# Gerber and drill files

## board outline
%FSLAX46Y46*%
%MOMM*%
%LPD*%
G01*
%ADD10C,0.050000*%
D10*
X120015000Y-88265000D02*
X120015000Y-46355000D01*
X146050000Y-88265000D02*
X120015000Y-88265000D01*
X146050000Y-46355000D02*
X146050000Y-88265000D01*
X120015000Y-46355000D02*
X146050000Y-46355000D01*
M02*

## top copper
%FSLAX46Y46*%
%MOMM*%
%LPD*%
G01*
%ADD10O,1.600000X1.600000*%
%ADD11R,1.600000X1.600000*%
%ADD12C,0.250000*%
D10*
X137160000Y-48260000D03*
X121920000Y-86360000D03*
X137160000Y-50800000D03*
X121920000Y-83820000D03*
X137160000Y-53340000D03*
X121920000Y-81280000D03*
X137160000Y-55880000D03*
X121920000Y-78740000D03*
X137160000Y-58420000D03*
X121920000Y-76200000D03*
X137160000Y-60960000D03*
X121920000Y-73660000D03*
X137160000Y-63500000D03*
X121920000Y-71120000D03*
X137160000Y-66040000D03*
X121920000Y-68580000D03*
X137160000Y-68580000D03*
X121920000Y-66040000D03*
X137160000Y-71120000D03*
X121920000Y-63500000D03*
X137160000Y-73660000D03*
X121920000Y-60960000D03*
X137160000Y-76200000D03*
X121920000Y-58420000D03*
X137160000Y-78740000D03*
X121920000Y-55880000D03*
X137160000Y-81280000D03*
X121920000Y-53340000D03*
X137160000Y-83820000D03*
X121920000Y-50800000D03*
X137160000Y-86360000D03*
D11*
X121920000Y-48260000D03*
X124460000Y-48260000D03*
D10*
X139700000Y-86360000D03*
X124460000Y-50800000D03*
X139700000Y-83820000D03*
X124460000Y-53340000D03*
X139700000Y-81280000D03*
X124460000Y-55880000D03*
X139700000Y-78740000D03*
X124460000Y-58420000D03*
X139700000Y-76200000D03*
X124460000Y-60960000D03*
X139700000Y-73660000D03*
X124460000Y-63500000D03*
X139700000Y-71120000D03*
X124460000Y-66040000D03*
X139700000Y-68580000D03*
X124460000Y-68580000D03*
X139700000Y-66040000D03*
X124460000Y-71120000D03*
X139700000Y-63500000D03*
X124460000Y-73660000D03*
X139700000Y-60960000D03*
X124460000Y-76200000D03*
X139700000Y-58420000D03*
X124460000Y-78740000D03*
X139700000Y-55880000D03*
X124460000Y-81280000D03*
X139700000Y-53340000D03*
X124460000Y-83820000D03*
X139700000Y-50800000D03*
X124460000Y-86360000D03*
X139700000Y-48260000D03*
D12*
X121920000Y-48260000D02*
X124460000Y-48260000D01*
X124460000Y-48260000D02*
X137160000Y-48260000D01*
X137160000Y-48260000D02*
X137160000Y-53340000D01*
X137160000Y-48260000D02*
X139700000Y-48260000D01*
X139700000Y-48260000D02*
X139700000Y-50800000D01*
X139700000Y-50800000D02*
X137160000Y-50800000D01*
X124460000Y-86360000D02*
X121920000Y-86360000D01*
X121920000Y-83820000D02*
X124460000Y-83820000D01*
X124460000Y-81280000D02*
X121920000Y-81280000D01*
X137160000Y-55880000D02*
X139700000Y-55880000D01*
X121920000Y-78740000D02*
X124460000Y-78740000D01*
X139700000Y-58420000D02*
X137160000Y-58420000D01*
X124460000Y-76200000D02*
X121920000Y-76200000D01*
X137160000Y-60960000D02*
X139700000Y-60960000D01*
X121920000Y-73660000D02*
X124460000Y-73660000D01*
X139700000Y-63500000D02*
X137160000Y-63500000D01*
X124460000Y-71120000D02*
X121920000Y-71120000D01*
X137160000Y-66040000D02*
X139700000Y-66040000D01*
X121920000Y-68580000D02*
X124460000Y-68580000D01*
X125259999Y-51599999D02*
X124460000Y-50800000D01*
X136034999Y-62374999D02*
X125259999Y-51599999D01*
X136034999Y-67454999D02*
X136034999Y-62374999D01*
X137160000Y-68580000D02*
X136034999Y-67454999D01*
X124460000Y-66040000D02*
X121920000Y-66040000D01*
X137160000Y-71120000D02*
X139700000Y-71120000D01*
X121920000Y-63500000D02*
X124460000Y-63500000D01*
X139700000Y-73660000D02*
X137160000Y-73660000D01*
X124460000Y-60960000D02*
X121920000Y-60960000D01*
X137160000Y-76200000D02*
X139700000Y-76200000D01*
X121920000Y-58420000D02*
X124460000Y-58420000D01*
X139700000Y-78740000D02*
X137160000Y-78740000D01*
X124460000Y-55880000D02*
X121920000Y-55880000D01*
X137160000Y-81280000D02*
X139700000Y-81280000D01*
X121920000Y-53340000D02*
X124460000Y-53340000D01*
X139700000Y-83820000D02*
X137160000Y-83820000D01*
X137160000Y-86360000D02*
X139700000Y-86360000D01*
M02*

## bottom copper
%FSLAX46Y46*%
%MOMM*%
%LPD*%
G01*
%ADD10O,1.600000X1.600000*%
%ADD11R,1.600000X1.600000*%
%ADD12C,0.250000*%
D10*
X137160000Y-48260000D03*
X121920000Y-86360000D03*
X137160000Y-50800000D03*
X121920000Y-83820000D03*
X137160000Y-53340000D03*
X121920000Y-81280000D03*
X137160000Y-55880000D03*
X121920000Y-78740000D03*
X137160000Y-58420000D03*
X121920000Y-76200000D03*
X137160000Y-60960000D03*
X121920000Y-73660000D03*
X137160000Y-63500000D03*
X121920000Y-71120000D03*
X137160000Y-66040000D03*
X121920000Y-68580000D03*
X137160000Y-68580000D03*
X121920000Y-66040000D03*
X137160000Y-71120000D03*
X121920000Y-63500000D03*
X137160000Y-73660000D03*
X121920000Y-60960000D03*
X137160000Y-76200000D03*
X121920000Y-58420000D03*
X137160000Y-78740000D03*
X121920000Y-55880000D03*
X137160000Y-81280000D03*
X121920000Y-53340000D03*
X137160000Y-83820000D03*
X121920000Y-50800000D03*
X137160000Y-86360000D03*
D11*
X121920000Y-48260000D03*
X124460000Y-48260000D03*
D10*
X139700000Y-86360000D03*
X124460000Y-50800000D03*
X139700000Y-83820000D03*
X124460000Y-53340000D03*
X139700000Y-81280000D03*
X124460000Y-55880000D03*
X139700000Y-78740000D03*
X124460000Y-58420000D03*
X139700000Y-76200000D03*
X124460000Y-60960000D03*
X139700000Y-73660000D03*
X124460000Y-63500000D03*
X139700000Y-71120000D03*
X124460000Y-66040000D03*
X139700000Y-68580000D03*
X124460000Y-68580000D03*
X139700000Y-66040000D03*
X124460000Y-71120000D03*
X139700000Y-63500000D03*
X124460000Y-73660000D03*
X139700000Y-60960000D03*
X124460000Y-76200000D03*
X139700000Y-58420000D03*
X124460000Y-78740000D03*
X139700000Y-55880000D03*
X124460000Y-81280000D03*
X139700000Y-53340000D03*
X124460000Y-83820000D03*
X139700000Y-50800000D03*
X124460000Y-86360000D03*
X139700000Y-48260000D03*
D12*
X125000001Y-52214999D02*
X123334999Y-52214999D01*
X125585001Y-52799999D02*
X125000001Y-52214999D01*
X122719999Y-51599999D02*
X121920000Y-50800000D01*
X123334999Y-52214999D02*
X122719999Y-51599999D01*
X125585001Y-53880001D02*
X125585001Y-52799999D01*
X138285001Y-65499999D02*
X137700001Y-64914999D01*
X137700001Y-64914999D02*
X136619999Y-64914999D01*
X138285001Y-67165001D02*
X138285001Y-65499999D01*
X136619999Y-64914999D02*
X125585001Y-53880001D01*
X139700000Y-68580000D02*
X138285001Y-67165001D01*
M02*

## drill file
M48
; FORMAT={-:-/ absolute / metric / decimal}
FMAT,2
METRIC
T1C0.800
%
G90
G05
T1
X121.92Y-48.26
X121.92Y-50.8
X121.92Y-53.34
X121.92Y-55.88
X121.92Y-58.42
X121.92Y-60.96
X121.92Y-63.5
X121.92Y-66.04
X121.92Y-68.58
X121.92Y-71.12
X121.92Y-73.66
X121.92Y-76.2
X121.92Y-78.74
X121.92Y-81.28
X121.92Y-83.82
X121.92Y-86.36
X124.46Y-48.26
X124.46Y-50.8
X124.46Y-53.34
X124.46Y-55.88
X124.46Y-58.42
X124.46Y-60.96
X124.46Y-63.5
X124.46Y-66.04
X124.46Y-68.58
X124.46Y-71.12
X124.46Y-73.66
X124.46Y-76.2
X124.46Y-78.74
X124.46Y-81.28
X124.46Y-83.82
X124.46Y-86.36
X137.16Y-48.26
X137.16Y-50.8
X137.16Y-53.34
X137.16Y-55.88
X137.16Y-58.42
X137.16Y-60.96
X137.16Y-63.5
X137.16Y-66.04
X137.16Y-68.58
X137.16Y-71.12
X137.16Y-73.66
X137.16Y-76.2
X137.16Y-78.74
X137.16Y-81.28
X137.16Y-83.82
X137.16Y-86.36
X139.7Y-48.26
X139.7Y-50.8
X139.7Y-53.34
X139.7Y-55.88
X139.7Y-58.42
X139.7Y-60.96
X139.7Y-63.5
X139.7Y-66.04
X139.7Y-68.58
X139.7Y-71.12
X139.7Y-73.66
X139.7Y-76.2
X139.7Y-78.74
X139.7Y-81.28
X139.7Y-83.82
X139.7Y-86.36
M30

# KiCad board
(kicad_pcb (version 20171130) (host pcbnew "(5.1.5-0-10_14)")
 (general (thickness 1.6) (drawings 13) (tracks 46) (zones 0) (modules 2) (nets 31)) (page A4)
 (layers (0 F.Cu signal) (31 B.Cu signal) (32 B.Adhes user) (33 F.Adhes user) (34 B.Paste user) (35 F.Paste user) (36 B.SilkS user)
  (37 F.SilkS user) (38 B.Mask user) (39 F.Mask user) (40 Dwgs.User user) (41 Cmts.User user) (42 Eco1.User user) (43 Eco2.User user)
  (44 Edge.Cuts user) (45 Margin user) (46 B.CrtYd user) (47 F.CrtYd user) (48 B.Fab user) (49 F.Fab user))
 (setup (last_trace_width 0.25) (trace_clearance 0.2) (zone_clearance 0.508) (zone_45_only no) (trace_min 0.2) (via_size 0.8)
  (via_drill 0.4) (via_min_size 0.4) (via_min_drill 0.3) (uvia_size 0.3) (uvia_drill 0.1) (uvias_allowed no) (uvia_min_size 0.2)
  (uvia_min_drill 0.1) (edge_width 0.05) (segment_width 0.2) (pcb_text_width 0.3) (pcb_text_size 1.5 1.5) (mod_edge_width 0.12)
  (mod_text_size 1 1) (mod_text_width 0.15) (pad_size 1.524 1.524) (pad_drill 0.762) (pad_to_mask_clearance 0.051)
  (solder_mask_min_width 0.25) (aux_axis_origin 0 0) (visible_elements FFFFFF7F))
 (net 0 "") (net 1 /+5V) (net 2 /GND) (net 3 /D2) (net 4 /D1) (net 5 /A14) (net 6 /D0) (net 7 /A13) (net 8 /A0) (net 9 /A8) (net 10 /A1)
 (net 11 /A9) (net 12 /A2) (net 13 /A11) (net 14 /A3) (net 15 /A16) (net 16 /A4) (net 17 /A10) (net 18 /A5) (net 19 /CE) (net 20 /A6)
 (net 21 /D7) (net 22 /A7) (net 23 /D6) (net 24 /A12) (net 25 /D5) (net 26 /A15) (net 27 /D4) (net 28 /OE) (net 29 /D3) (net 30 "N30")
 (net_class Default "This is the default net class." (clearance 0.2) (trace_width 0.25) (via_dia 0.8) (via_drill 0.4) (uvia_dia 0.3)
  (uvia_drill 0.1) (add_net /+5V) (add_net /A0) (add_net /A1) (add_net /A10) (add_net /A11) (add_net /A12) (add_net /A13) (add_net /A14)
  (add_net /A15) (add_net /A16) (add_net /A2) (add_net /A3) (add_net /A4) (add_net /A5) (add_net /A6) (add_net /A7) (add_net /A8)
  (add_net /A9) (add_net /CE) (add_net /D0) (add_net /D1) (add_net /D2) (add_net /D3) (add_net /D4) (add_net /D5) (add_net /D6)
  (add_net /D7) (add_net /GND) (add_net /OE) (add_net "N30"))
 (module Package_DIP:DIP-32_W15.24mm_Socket (layer F.Cu) (at 121.92 48.26)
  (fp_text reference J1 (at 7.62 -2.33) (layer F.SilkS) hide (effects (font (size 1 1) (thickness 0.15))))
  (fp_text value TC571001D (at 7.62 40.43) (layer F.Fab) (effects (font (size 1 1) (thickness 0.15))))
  (pad 32 thru_hole oval (at 15.24 0) (size 1.6 1.6) (drill 0.8) (layers *.Cu *.Mask) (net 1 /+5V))
  (pad 16 thru_hole oval (at 0 38.1) (size 1.6 1.6) (drill 0.8) (layers *.Cu *.Mask) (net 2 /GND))
  (pad 31 thru_hole oval (at 15.24 2.54) (size 1.6 1.6) (drill 0.8) (layers *.Cu *.Mask) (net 1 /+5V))
  (pad 15 thru_hole oval (at 0 35.56) (size 1.6 1.6) (drill 0.8) (layers *.Cu *.Mask) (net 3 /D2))
  (pad 30 thru_hole oval (at 15.24 5.08) (size 1.6 1.6) (drill 0.8) (layers *.Cu *.Mask) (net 1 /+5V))
  (pad 14 thru_hole oval (at 0 33.02) (size 1.6 1.6) (drill 0.8) (layers *.Cu *.Mask) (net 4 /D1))
  (pad 29 thru_hole oval (at 15.24 7.62) (size 1.6 1.6) (drill 0.8) (layers *.Cu *.Mask) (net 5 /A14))
  (pad 13 thru_hole oval (at 0 30.48) (size 1.6 1.6) (drill 0.8) (layers *.Cu *.Mask) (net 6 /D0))
  (pad 28 thru_hole oval (at 15.24 10.16) (size 1.6 1.6) (drill 0.8) (layers *.Cu *.Mask) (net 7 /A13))
  (pad 12 thru_hole oval (at 0 27.94) (size 1.6 1.6) (drill 0.8) (layers *.Cu *.Mask) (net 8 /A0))
  (pad 27 thru_hole oval (at 15.24 12.7) (size 1.6 1.6) (drill 0.8) (layers *.Cu *.Mask) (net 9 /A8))
  (pad 11 thru_hole oval (at 0 25.4) (size 1.6 1.6) (drill 0.8) (layers *.Cu *.Mask) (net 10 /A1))
  (pad 26 thru_hole oval (at 15.24 15.24) (size 1.6 1.6) (drill 0.8) (layers *.Cu *.Mask) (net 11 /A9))
  (pad 10 thru_hole oval (at 0 22.86) (size 1.6 1.6) (drill 0.8) (layers *.Cu *.Mask) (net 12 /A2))
  (pad 25 thru_hole oval (at 15.24 17.78) (size 1.6 1.6) (drill 0.8) (layers *.Cu *.Mask) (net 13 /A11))
  (pad 9 thru_hole oval (at 0 20.32) (size 1.6 1.6) (drill 0.8) (layers *.Cu *.Mask) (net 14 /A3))
  (pad 24 thru_hole oval (at 15.24 20.32) (size 1.6 1.6) (drill 0.8) (layers *.Cu *.Mask) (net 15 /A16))
  (pad 8 thru_hole oval (at 0 17.78) (size 1.6 1.6) (drill 0.8) (layers *.Cu *.Mask) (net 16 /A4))
  (pad 23 thru_hole oval (at 15.24 22.86) (size 1.6 1.6) (drill 0.8) (layers *.Cu *.Mask) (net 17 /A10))
  (pad 7 thru_hole oval (at 0 15.24) (size 1.6 1.6) (drill 0.8) (layers *.Cu *.Mask) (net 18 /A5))
  (pad 22 thru_hole oval (at 15.24 25.4) (size 1.6 1.6) (drill 0.8) (layers *.Cu *.Mask) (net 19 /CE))
  (pad 6 thru_hole oval (at 0 12.7) (size 1.6 1.6) (drill 0.8) (layers *.Cu *.Mask) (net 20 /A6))
  (pad 21 thru_hole oval (at 15.24 27.94) (size 1.6 1.6) (drill 0.8) (layers *.Cu *.Mask) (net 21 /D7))
  (pad 5 thru_hole oval (at 0 10.16) (size 1.6 1.6) (drill 0.8) (layers *.Cu *.Mask) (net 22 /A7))
  (pad 20 thru_hole oval (at 15.24 30.48) (size 1.6 1.6) (drill 0.8) (layers *.Cu *.Mask) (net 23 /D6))
  (pad 4 thru_hole oval (at 0 7.62) (size 1.6 1.6) (drill 0.8) (layers *.Cu *.Mask) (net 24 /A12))
  (pad 19 thru_hole oval (at 15.24 33.02) (size 1.6 1.6) (drill 0.8) (layers *.Cu *.Mask) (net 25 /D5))
  (pad 3 thru_hole oval (at 0 5.08) (size 1.6 1.6) (drill 0.8) (layers *.Cu *.Mask) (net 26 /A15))
  (pad 18 thru_hole oval (at 15.24 35.56) (size 1.6 1.6) (drill 0.8) (layers *.Cu *.Mask) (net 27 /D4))
  (pad 2 thru_hole oval (at 0 2.54) (size 1.6 1.6) (drill 0.8) (layers *.Cu *.Mask) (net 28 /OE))
  (pad 17 thru_hole oval (at 15.24 38.1) (size 1.6 1.6) (drill 0.8) (layers *.Cu *.Mask) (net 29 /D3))
  (pad 1 thru_hole rect (at 0 0) (size 1.6 1.6) (drill 0.8) (layers *.Cu *.Mask) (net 1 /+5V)))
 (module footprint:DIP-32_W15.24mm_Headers (layer B.Cu) (at 139.7 48.26 180)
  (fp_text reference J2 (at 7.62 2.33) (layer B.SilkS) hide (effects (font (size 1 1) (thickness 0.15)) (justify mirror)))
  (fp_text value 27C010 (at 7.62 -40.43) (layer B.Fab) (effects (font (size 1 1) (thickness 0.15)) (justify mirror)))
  (pad 1 thru_hole rect (at 15.24 0 180) (size 1.6 1.6) (drill 0.8) (layers *.Cu *.Mask) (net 1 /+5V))
  (pad 17 thru_hole oval (at 0 -38.1 180) (size 1.6 1.6) (drill 0.8) (layers *.Cu *.Mask) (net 29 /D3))
  (pad 2 thru_hole oval (at 15.24 -2.54 180) (size 1.6 1.6) (drill 0.8) (layers *.Cu *.Mask) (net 15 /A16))
  (pad 18 thru_hole oval (at 0 -35.56 180) (size 1.6 1.6) (drill 0.8) (layers *.Cu *.Mask) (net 27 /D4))
  (pad 3 thru_hole oval (at 15.24 -5.08 180) (size 1.6 1.6) (drill 0.8) (layers *.Cu *.Mask) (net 26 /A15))
  (pad 19 thru_hole oval (at 0 -33.02 180) (size 1.6 1.6) (drill 0.8) (layers *.Cu *.Mask) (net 25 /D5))
  (pad 4 thru_hole oval (at 15.24 -7.62 180) (size 1.6 1.6) (drill 0.8) (layers *.Cu *.Mask) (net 24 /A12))
  (pad 20 thru_hole oval (at 0 -30.48 180) (size 1.6 1.6) (drill 0.8) (layers *.Cu *.Mask) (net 23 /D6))
  (pad 5 thru_hole oval (at 15.24 -10.16 180) (size 1.6 1.6) (drill 0.8) (layers *.Cu *.Mask) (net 22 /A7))
  (pad 21 thru_hole oval (at 0 -27.94 180) (size 1.6 1.6) (drill 0.8) (layers *.Cu *.Mask) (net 21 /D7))
  (pad 6 thru_hole oval (at 15.24 -12.7 180) (size 1.6 1.6) (drill 0.8) (layers *.Cu *.Mask) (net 20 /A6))
  (pad 22 thru_hole oval (at 0 -25.4 180) (size 1.6 1.6) (drill 0.8) (layers *.Cu *.Mask) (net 19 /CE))
  (pad 7 thru_hole oval (at 15.24 -15.24 180) (size 1.6 1.6) (drill 0.8) (layers *.Cu *.Mask) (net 18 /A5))
  (pad 23 thru_hole oval (at 0 -22.86 180) (size 1.6 1.6) (drill 0.8) (layers *.Cu *.Mask) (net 17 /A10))
  (pad 8 thru_hole oval (at 15.24 -17.78 180) (size 1.6 1.6) (drill 0.8) (layers *.Cu *.Mask) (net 16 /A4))
  (pad 24 thru_hole oval (at 0 -20.32 180) (size 1.6 1.6) (drill 0.8) (layers *.Cu *.Mask) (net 28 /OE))
  (pad 9 thru_hole oval (at 15.24 -20.32 180) (size 1.6 1.6) (drill 0.8) (layers *.Cu *.Mask) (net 14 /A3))
  (pad 25 thru_hole oval (at 0 -17.78 180) (size 1.6 1.6) (drill 0.8) (layers *.Cu *.Mask) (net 13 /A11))
  (pad 10 thru_hole oval (at 15.24 -22.86 180) (size 1.6 1.6) (drill 0.8) (layers *.Cu *.Mask) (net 12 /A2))
  (pad 26 thru_hole oval (at 0 -15.24 180) (size 1.6 1.6) (drill 0.8) (layers *.Cu *.Mask) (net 11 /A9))
  (pad 11 thru_hole oval (at 15.24 -25.4 180) (size 1.6 1.6) (drill 0.8) (layers *.Cu *.Mask) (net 10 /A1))
  (pad 27 thru_hole oval (at 0 -12.7 180) (size 1.6 1.6) (drill 0.8) (layers *.Cu *.Mask) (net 9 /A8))
  (pad 12 thru_hole oval (at 15.24 -27.94 180) (size 1.6 1.6) (drill 0.8) (layers *.Cu *.Mask) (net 8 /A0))
  (pad 28 thru_hole oval (at 0 -10.16 180) (size 1.6 1.6) (drill 0.8) (layers *.Cu *.Mask) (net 7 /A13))
  (pad 13 thru_hole oval (at 15.24 -30.48 180) (size 1.6 1.6) (drill 0.8) (layers *.Cu *.Mask) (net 6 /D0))
  (pad 29 thru_hole oval (at 0 -7.62 180) (size 1.6 1.6) (drill 0.8) (layers *.Cu *.Mask) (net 5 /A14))
  (pad 14 thru_hole oval (at 15.24 -33.02 180) (size 1.6 1.6) (drill 0.8) (layers *.Cu *.Mask) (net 4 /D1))
  (pad 30 thru_hole oval (at 0 -5.08 180) (size 1.6 1.6) (drill 0.8) (layers *.Cu *.Mask) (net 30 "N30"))
  (pad 15 thru_hole oval (at 15.24 -35.56 180) (size 1.6 1.6) (drill 0.8) (layers *.Cu *.Mask) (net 3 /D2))
  (pad 31 thru_hole oval (at 0 -2.54 180) (size 1.6 1.6) (drill 0.8) (layers *.Cu *.Mask) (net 1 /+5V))
  (pad 16 thru_hole oval (at 15.24 -38.1 180) (size 1.6 1.6) (drill 0.8) (layers *.Cu *.Mask) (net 2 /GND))
  (pad 32 thru_hole oval (at 0 0 180) (size 1.6 1.6) (drill 0.8) (layers *.Cu *.Mask) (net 1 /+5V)))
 (gr_line (start 120.015 88.265) (end 120.015 46.355) (layer Edge.Cuts) (width 0.05))
 (gr_line (start 146.05 88.265) (end 120.015 88.265) (layer Edge.Cuts) (width 0.05))
 (gr_line (start 146.05 46.355) (end 146.05 88.265) (layer Edge.Cuts) (width 0.05))
 (gr_line (start 120.015 46.355) (end 146.05 46.355) (layer Edge.Cuts) (width 0.05))
 (segment (start 121.92 48.26) (end 124.46 48.26) (width 0.25) (layer F.Cu) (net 1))
 (segment (start 124.46 48.26) (end 137.16 48.26) (width 0.25) (layer F.Cu) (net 1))
 (segment (start 137.16 48.26) (end 137.16 53.34) (width 0.25) (layer F.Cu) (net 1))
 (segment (start 137.16 48.26) (end 139.7 48.26) (width 0.25) (layer F.Cu) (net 1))
 (segment (start 139.7 48.26) (end 139.7 50.8) (width 0.25) (layer F.Cu) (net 1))
 (segment (start 139.7 50.8) (end 137.16 50.8) (width 0.25) (layer F.Cu) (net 1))
 (segment (start 124.46 86.36) (end 121.92 86.36) (width 0.25) (layer F.Cu) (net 2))
 (segment (start 121.92 83.82) (end 124.46 83.82) (width 0.25) (layer F.Cu) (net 3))
 (segment (start 124.46 81.28) (end 121.92 81.28) (width 0.25) (layer F.Cu) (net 4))
 (segment (start 137.16 55.88) (end 139.7 55.88) (width 0.25) (layer F.Cu) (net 5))
 (segment (start 121.92 78.74) (end 124.46 78.74) (width 0.25) (layer F.Cu) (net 6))
 (segment (start 139.7 58.42) (end 137.16 58.42) (width 0.25) (layer F.Cu) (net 7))
 (segment (start 124.46 76.2) (end 121.92 76.2) (width 0.25) (layer F.Cu) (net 8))
 (segment (start 137.16 60.96) (end 139.7 60.96) (width 0.25) (layer F.Cu) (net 9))
 (segment (start 121.92 73.66) (end 124.46 73.66) (width 0.25) (layer F.Cu) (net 10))
 (segment (start 139.7 63.5) (end 137.16 63.5) (width 0.25) (layer F.Cu) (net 11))
 (segment (start 124.46 71.12) (end 121.92 71.12) (width 0.25) (layer F.Cu) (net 12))
 (segment (start 137.16 66.04) (end 139.7 66.04) (width 0.25) (layer F.Cu) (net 13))
 (segment (start 121.92 68.58) (end 124.46 68.58) (width 0.25) (layer F.Cu) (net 14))
 (segment (start 125.259999 51.599999) (end 124.46 50.8) (width 0.25) (layer F.Cu) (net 15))
 (segment (start 136.034999 62.374999) (end 125.259999 51.599999) (width 0.25) (layer F.Cu) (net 15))
 (segment (start 136.034999 67.454999) (end 136.034999 62.374999) (width 0.25) (layer F.Cu) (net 15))
 (segment (start 137.16 68.58) (end 136.034999 67.454999) (width 0.25) (layer F.Cu) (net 15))
 (segment (start 124.46 66.04) (end 121.92 66.04) (width 0.25) (layer F.Cu) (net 16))
 (segment (start 137.16 71.12) (end 139.7 71.12) (width 0.25) (layer F.Cu) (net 17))
 (segment (start 121.92 63.5) (end 124.46 63.5) (width 0.25) (layer F.Cu) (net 18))
 (segment (start 139.7 73.66) (end 137.16 73.66) (width 0.25) (layer F.Cu) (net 19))
 (segment (start 124.46 60.96) (end 121.92 60.96) (width 0.25) (layer F.Cu) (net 20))
 (segment (start 137.16 76.2) (end 139.7 76.2) (width 0.25) (layer F.Cu) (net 21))
 (segment (start 121.92 58.42) (end 124.46 58.42) (width 0.25) (layer F.Cu) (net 22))
 (segment (start 139.7 78.74) (end 137.16 78.74) (width 0.25) (layer F.Cu) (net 23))
 (segment (start 124.46 55.88) (end 121.92 55.88) (width 0.25) (layer F.Cu) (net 24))
 (segment (start 137.16 81.28) (end 139.7 81.28) (width 0.25) (layer F.Cu) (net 25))
 (segment (start 121.92 53.34) (end 124.46 53.34) (width 0.25) (layer F.Cu) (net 26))
 (segment (start 139.7 83.82) (end 137.16 83.82) (width 0.25) (layer F.Cu) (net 27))
 (segment (start 125.000001 52.214999) (end 123.334999 52.214999) (width 0.25) (layer B.Cu) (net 28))
 (segment (start 125.585001 52.799999) (end 125.000001 52.214999) (width 0.25) (layer B.Cu) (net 28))
 (segment (start 122.719999 51.599999) (end 121.92 50.8) (width 0.25) (layer B.Cu) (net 28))
 (segment (start 123.334999 52.214999) (end 122.719999 51.599999) (width 0.25) (layer B.Cu) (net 28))
 (segment (start 125.585001 53.880001) (end 125.585001 52.799999) (width 0.25) (layer B.Cu) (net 28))
 (segment (start 138.285001 65.499999) (end 137.700001 64.914999) (width 0.25) (layer B.Cu) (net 28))
 (segment (start 137.700001 64.914999) (end 136.619999 64.914999) (width 0.25) (layer B.Cu) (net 28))
 (segment (start 138.285001 67.165001) (end 138.285001 65.499999) (width 0.25) (layer B.Cu) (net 28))
 (segment (start 136.619999 64.914999) (end 125.585001 53.880001) (width 0.25) (layer B.Cu) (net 28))
 (segment (start 139.7 68.58) (end 138.285001 67.165001) (width 0.25) (layer B.Cu) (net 28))
 (segment (start 137.16 86.36) (end 139.7 86.36) (width 0.25) (layer F.Cu) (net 29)))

